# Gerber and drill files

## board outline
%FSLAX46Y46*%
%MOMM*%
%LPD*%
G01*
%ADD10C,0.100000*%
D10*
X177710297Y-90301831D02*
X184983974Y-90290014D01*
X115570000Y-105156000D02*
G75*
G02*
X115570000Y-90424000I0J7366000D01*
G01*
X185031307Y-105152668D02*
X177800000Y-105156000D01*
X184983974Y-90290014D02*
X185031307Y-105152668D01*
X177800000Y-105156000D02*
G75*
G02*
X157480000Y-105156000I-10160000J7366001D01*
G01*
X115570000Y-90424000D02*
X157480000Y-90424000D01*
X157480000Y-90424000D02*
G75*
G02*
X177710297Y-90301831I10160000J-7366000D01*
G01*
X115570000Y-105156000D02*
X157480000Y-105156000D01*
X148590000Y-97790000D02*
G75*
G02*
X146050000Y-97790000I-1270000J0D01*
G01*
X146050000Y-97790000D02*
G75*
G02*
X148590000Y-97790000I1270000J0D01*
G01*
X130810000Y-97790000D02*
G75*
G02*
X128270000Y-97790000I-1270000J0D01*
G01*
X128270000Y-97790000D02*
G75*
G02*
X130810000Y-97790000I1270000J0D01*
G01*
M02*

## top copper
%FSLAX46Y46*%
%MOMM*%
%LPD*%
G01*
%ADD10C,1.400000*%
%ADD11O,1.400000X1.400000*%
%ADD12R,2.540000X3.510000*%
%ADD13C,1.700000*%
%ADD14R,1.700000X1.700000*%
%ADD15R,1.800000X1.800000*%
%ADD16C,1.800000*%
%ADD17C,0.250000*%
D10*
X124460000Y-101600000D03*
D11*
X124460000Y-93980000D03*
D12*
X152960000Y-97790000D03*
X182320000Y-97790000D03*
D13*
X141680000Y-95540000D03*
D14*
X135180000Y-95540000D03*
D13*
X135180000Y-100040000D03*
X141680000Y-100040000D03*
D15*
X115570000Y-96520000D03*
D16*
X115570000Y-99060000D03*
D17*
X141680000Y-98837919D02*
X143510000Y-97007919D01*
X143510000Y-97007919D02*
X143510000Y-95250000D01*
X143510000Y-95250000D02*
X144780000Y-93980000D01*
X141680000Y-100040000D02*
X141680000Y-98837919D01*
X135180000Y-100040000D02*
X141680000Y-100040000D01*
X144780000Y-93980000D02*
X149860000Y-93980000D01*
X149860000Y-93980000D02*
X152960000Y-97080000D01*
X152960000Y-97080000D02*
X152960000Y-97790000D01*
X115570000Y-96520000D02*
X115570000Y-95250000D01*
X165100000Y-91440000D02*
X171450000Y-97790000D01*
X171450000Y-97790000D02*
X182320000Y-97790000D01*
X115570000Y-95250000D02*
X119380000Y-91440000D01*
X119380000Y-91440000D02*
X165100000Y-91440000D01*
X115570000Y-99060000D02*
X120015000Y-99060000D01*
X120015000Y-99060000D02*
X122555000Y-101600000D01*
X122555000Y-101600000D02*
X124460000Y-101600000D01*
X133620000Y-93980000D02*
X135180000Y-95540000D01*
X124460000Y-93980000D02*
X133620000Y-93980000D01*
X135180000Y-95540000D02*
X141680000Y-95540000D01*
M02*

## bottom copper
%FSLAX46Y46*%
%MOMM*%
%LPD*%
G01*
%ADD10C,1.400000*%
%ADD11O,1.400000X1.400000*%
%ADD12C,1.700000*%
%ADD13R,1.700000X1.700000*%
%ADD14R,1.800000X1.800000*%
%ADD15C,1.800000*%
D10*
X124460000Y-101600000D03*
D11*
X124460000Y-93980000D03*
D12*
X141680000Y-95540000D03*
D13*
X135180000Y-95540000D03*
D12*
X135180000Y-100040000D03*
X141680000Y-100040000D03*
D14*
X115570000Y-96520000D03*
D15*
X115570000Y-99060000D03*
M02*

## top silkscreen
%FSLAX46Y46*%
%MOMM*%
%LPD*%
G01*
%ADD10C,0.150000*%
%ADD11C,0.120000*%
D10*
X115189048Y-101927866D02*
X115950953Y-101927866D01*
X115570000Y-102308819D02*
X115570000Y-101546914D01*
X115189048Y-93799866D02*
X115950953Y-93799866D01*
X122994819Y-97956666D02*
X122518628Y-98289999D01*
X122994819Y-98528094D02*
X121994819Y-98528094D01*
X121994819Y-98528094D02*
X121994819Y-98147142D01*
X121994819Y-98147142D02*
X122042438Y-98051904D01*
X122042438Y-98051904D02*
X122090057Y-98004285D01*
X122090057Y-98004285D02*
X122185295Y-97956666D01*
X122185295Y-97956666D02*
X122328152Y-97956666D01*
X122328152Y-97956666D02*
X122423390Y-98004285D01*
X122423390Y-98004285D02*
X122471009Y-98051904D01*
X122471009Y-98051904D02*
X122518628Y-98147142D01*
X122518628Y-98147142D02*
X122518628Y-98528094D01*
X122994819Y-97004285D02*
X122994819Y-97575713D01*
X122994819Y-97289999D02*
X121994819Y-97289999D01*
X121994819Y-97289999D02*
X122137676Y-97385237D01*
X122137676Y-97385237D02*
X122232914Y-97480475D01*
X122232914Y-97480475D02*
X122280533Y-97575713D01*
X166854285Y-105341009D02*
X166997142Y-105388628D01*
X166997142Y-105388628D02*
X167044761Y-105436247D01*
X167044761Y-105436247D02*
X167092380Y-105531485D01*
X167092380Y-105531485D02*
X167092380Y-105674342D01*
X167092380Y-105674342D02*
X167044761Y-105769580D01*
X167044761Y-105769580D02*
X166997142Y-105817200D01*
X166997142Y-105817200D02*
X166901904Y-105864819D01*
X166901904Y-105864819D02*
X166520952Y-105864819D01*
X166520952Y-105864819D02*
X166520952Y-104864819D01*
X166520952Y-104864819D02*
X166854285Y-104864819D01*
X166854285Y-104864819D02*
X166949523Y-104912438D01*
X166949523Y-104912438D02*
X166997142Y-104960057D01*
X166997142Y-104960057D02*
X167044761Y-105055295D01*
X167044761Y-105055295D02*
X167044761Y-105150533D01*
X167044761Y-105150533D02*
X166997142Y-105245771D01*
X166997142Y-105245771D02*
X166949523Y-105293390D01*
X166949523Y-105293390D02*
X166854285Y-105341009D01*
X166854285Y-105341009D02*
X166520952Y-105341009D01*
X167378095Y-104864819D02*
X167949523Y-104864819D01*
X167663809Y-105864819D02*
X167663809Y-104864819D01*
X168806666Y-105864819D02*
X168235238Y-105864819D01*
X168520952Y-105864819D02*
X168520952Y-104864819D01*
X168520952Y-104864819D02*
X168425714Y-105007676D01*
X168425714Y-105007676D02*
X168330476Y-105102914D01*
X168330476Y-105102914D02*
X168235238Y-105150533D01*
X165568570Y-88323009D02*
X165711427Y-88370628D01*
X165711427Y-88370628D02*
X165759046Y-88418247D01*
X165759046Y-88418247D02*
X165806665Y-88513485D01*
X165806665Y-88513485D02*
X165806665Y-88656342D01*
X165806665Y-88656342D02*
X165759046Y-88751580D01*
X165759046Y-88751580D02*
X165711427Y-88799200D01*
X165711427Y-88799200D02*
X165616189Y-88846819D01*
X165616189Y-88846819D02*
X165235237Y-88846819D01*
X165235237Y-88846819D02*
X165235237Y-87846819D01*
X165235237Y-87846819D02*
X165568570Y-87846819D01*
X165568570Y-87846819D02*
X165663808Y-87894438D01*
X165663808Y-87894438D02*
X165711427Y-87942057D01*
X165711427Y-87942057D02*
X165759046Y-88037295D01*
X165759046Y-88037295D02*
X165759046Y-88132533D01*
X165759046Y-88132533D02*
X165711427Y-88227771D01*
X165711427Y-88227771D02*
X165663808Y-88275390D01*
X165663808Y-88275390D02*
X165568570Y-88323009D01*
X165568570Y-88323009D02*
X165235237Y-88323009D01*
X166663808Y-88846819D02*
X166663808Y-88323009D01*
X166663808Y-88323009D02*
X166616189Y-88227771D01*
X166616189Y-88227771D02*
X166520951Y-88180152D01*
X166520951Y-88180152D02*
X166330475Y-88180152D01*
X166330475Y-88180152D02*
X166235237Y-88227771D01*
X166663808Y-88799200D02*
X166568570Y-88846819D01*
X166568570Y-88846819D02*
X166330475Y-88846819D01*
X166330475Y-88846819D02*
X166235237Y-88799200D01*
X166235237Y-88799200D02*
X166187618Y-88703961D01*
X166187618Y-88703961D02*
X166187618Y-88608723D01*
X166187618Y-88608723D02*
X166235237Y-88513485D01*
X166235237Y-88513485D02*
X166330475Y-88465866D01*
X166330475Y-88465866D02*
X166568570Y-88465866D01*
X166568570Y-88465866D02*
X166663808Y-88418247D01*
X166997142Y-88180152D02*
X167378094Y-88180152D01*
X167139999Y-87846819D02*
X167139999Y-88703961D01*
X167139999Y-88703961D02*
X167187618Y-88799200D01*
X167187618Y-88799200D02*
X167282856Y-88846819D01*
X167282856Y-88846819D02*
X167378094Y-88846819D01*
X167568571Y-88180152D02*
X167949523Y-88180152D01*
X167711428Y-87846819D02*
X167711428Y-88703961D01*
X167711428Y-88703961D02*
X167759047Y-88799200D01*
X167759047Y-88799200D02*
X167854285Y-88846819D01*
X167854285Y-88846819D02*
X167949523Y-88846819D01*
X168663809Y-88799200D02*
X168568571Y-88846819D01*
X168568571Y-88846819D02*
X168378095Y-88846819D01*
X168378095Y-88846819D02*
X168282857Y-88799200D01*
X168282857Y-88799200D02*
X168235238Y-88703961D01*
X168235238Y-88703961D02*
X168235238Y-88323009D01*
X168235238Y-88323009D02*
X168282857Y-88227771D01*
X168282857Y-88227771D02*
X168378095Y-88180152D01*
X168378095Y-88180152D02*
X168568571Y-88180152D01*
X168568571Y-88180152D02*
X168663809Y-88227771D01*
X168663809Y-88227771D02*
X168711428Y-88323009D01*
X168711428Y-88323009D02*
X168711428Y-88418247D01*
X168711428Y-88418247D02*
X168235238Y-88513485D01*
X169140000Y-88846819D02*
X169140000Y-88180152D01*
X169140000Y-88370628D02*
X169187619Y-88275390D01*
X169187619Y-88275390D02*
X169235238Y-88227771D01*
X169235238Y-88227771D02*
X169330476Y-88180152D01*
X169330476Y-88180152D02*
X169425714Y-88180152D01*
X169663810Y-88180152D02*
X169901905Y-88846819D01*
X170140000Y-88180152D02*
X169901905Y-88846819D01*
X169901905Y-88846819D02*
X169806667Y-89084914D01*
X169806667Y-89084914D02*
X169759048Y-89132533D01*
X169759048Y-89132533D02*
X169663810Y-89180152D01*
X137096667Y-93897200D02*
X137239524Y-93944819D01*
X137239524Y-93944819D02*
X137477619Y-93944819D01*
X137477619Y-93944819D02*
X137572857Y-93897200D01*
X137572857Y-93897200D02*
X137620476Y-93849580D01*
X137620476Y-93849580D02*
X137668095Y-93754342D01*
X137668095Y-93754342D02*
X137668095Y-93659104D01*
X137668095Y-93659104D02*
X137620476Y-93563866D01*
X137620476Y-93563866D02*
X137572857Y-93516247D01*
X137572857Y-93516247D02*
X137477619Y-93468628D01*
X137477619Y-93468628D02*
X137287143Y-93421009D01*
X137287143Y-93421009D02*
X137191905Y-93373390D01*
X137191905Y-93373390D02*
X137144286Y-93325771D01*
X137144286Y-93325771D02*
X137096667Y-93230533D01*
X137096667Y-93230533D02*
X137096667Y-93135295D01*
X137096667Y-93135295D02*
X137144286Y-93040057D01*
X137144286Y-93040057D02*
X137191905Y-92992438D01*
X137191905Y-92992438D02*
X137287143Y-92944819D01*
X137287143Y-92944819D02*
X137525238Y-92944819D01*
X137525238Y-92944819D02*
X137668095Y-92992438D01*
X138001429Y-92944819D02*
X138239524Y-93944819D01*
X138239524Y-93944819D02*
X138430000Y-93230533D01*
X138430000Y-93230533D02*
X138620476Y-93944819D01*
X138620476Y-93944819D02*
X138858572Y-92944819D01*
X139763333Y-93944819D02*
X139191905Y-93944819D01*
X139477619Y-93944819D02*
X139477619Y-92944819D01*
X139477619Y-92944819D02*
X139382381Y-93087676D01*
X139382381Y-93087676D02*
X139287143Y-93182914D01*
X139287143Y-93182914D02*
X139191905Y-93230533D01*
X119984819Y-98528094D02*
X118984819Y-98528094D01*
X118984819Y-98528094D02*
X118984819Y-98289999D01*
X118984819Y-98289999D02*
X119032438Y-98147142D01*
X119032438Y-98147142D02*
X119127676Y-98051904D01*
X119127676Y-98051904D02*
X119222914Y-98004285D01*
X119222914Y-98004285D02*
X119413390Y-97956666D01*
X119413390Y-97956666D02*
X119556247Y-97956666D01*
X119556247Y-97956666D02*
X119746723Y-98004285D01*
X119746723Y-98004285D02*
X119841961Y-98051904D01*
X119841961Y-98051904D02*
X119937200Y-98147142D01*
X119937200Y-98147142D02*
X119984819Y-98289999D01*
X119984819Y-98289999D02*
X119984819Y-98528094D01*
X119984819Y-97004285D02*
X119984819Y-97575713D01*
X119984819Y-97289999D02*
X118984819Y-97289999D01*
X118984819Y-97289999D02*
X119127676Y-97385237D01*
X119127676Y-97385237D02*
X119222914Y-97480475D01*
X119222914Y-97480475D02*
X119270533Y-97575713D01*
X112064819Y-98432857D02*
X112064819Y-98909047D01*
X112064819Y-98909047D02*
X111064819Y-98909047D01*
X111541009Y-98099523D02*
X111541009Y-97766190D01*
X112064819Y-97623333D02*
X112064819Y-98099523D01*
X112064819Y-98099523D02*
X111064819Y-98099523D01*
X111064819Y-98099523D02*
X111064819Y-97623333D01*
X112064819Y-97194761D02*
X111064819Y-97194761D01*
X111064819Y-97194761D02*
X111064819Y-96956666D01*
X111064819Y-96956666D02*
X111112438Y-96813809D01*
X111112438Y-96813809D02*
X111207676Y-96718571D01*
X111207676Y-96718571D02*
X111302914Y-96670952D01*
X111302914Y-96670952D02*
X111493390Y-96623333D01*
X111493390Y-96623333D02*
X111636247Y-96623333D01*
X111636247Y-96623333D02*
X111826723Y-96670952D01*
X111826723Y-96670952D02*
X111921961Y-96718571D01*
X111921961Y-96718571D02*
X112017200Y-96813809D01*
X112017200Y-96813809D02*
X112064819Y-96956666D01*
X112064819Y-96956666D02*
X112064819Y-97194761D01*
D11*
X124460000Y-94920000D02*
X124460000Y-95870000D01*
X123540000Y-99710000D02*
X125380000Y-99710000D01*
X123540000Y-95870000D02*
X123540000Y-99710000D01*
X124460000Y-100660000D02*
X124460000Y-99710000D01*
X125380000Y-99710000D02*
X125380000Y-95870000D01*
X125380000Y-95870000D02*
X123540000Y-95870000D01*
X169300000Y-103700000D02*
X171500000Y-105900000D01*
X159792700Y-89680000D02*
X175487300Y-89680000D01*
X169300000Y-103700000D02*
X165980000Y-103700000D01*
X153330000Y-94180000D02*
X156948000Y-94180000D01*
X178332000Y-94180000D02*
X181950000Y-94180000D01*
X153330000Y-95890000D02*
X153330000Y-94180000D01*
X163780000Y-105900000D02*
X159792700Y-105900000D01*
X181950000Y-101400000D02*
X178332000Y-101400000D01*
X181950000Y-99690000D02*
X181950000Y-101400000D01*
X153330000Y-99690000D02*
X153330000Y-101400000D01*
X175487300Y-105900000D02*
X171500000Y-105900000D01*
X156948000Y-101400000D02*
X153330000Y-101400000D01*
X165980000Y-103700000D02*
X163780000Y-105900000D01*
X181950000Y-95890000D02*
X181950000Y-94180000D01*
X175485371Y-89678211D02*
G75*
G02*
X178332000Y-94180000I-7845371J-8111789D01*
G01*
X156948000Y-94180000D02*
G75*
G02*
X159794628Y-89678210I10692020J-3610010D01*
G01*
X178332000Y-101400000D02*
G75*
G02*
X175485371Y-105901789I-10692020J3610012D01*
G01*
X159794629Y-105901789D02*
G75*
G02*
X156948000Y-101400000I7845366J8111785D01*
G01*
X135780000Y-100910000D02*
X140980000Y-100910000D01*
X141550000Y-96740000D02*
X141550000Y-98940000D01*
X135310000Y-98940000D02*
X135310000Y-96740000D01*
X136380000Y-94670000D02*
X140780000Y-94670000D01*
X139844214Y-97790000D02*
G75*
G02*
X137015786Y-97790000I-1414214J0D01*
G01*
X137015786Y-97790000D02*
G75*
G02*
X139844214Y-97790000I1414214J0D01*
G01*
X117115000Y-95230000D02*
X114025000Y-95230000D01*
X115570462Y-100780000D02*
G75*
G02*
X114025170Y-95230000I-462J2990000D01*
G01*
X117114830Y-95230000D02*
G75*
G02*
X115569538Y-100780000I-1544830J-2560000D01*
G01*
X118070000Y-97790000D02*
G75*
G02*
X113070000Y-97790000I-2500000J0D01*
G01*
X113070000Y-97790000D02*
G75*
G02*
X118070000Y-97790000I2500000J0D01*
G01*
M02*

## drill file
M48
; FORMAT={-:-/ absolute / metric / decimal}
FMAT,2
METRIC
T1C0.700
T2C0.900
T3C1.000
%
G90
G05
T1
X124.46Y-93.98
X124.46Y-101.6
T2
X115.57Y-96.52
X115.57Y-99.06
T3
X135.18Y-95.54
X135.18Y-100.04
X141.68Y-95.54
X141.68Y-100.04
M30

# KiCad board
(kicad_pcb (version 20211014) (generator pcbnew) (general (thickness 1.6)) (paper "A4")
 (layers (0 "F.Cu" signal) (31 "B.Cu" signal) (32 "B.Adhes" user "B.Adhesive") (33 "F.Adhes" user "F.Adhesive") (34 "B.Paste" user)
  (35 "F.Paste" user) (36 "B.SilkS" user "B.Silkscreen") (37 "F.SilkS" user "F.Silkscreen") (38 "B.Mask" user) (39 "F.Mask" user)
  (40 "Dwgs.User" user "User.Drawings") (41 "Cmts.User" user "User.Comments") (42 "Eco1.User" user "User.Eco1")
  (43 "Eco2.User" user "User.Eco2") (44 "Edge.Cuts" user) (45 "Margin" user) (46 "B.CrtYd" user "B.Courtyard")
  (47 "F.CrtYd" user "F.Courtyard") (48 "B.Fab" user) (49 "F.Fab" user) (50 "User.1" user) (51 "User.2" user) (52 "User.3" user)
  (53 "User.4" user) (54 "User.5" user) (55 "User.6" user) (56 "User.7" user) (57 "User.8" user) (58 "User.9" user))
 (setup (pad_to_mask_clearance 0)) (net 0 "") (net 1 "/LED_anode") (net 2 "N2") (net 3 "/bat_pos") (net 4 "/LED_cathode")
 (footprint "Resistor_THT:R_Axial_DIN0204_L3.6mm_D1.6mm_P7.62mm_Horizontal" (layer "F.Cu") (at 124.46 101.6 90)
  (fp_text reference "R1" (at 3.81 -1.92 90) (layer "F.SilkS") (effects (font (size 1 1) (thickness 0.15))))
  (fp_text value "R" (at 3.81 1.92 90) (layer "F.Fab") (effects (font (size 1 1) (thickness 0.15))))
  (fp_line (start 6.68 0) (end 5.73 0) (layer "F.SilkS") (width 0.12))
  (fp_line (start 1.89 -0.92) (end 1.89 0.92) (layer "F.SilkS") (width 0.12))
  (fp_line (start 5.73 -0.92) (end 1.89 -0.92) (layer "F.SilkS") (width 0.12))
  (fp_line (start 0.94 0) (end 1.89 0) (layer "F.SilkS") (width 0.12))
  (fp_line (start 1.89 0.92) (end 5.73 0.92) (layer "F.SilkS") (width 0.12))
  (fp_line (start 5.73 0.92) (end 5.73 -0.92) (layer "F.SilkS") (width 0.12))
  (pad "1" thru_hole circle (at 0 0 90) (size 1.4 1.4) (drill 0.7) (layers *.Cu *.Mask) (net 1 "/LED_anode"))
  (pad "2" thru_hole oval (at 7.62 0 90) (size 1.4 1.4) (drill 0.7) (layers *.Cu *.Mask) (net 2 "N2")))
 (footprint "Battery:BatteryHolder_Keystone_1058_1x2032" (layer "F.Cu") (at 167.64 97.79)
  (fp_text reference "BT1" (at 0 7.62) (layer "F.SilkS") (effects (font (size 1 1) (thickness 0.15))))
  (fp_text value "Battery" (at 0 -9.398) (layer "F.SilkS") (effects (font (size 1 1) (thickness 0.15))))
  (fp_line (start 1.66 5.91) (end 3.86 8.11) (layer "F.SilkS") (width 0.12))
  (fp_line (start -7.8473 -8.11) (end 7.8473 -8.11) (layer "F.SilkS") (width 0.12))
  (fp_line (start 1.66 5.91) (end -1.66 5.91) (layer "F.SilkS") (width 0.12))
  (fp_line (start -14.31 -3.61) (end -10.692 -3.61) (layer "F.SilkS") (width 0.12))
  (fp_line (start 10.692 -3.61) (end 14.31 -3.61) (layer "F.SilkS") (width 0.12))
  (fp_line (start -14.31 -1.9) (end -14.31 -3.61) (layer "F.SilkS") (width 0.12))
  (fp_line (start -3.86 8.11) (end -7.8473 8.11) (layer "F.SilkS") (width 0.12))
  (fp_line (start 14.31 3.61) (end 10.692 3.61) (layer "F.SilkS") (width 0.12))
  (fp_line (start 14.31 1.9) (end 14.31 3.61) (layer "F.SilkS") (width 0.12))
  (fp_line (start -14.31 1.9) (end -14.31 3.61) (layer "F.SilkS") (width 0.12))
  (fp_line (start 7.8473 8.11) (end 3.86 8.11) (layer "F.SilkS") (width 0.12))
  (fp_line (start -10.692 3.61) (end -14.31 3.61) (layer "F.SilkS") (width 0.12))
  (fp_line (start -1.66 5.91) (end -3.86 8.11) (layer "F.SilkS") (width 0.12))
  (fp_line (start 14.31 -1.9) (end 14.31 -3.61) (layer "F.SilkS") (width 0.12))
  (fp_arc (start 7.845371 -8.111789) (mid 9.538085 -6.031244) (end 10.692 -3.61) (layer "F.SilkS") (width 0.12))
  (fp_arc (start -10.692 -3.61) (mid -9.538084 -6.031244) (end -7.845371 -8.111789) (layer "F.SilkS") (width 0.12))
  (fp_arc (start 10.692 3.61) (mid 9.538084 6.031244) (end 7.845371 8.111789) (layer "F.SilkS") (width 0.12))
  (fp_arc (start -7.845371 8.111789) (mid -9.538085 6.031244) (end -10.692 3.61) (layer "F.SilkS") (width 0.12))
  (pad "1" smd rect (at -14.68 0) (size 2.54 3.51) (layers "F.Cu" "F.Paste" "F.Mask") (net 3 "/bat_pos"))
  (pad "2" smd rect (at 14.68 0) (size 2.54 3.51) (layers "F.Cu" "F.Paste" "F.Mask") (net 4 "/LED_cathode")))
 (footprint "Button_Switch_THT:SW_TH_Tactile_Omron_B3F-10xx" (layer "F.Cu") (at 135.18 95.54)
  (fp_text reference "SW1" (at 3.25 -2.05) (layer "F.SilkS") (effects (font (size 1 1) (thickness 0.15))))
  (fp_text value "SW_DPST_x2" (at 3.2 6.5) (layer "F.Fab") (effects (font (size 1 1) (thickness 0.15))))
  (fp_line (start 0.6 5.37) (end 5.8 5.37) (layer "F.SilkS") (width 0.12))
  (fp_line (start 6.37 1.2) (end 6.37 3.4) (layer "F.SilkS") (width 0.12))
  (fp_line (start 0.13 3.4) (end 0.13 1.2) (layer "F.SilkS") (width 0.12))
  (fp_line (start 1.2 -0.87) (end 5.6 -0.87) (layer "F.SilkS") (width 0.12))
  (fp_circle (center 3.25 2.25) (end 4.25 3.25) (layer "F.SilkS") (width 0.12) (fill none))
  (pad "1" thru_hole circle (at 6.5 0) (size 1.7 1.7) (drill 1) (layers *.Cu *.Mask) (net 2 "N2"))
  (pad "1" thru_hole rect (at 0 0) (size 1.7 1.7) (drill 1) (layers *.Cu *.Mask) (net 2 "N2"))
  (pad "2" thru_hole circle (at 0 4.5) (size 1.7 1.7) (drill 1) (layers *.Cu *.Mask) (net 3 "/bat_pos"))
  (pad "2" thru_hole circle (at 6.5 4.5) (size 1.7 1.7) (drill 1) (layers *.Cu *.Mask) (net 3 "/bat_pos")))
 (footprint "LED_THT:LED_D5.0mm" (layer "F.Cu") (at 115.57 96.52 -90)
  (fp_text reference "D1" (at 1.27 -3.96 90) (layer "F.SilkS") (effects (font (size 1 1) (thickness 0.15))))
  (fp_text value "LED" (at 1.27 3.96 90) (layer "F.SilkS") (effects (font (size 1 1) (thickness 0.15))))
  (fp_line (start -1.29 -1.545) (end -1.29 1.545) (layer "F.SilkS") (width 0.12))
  (fp_arc (start 4.26 -0.000462) (mid 2.072002 2.880433) (end -1.29 1.54483) (layer "F.SilkS") (width 0.12))
  (fp_arc (start -1.29 -1.54483) (mid 2.072002 -2.880433) (end 4.26 0.000462) (layer "F.SilkS") (width 0.12))
  (fp_circle (center 1.27 0) (end 3.77 0) (layer "F.SilkS") (width 0.12) (fill none))
  (pad "1" thru_hole rect (at 0 0 270) (size 1.8 1.8) (drill 0.9) (layers *.Cu *.Mask) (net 4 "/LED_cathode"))
  (pad "2" thru_hole circle (at 2.54 0 270) (size 1.8 1.8) (drill 0.9) (layers *.Cu *.Mask) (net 1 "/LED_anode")))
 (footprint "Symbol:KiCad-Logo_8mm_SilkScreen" (layer "B.Cu") (at 167.64 97.536 180)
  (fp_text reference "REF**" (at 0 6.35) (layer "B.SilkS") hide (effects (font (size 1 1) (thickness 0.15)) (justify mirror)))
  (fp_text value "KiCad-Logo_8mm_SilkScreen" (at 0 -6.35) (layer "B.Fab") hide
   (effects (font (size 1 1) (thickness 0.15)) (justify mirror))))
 (gr_line (start 177.710297 90.301831) (end 184.983974 90.290014) (layer "Edge.Cuts") (width 0.1))
 (gr_arc (start 115.57 105.156) (mid 108.204 97.79) (end 115.57 90.424) (layer "Edge.Cuts") (width 0.1))
 (gr_line (start 185.031307 105.152668) (end 177.8 105.156) (layer "Edge.Cuts") (width 0.1))
 (gr_line (start 184.983974 90.290014) (end 185.031307 105.152668) (layer "Edge.Cuts") (width 0.1))
 (gr_arc (start 177.8 105.156) (mid 167.64 110.339245) (end 157.48 105.156) (layer "Edge.Cuts") (width 0.1))
 (gr_line (start 115.57 90.424) (end 157.48 90.424) (layer "Edge.Cuts") (width 0.1))
 (gr_arc (start 157.48 90.424) (mid 167.564218 85.240984) (end 177.710297 90.301831) (layer "Edge.Cuts") (width 0.1))
 (gr_line (start 115.57 105.156) (end 157.48 105.156) (layer "Edge.Cuts") (width 0.1))
 (gr_circle (center 147.32 97.79) (end 146.05 97.79) (layer "Edge.Cuts") (width 0.1) (fill none))
 (gr_circle (center 129.54 97.79) (end 128.27 97.79) (layer "Edge.Cuts") (width 0.1) (fill none))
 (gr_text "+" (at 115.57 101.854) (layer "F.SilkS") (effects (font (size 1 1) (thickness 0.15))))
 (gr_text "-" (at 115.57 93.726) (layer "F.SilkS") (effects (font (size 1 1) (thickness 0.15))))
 (segment (start 141.68 98.837919) (end 143.51 97.007919) (width 0.25) (layer "F.Cu") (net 3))
 (segment (start 143.51 97.007919) (end 143.51 95.25) (width 0.25) (layer "F.Cu") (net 3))
 (segment (start 143.51 95.25) (end 144.78 93.98) (width 0.25) (layer "F.Cu") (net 3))
 (segment (start 141.68 100.04) (end 141.68 98.837919) (width 0.25) (layer "F.Cu") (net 3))
 (segment (start 135.18 100.04) (end 141.68 100.04) (width 0.25) (layer "F.Cu") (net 3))
 (segment (start 144.78 93.98) (end 149.86 93.98) (width 0.25) (layer "F.Cu") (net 3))
 (segment (start 149.86 93.98) (end 152.96 97.08) (width 0.25) (layer "F.Cu") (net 3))
 (segment (start 152.96 97.08) (end 152.96 97.79) (width 0.25) (layer "F.Cu") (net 3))
 (segment (start 115.57 96.52) (end 115.57 95.25) (width 0.25) (layer "F.Cu") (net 4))
 (segment (start 165.1 91.44) (end 171.45 97.79) (width 0.25) (layer "F.Cu") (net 4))
 (segment (start 171.45 97.79) (end 182.32 97.79) (width 0.25) (layer "F.Cu") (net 4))
 (segment (start 115.57 95.25) (end 119.38 91.44) (width 0.25) (layer "F.Cu") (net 4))
 (segment (start 119.38 91.44) (end 165.1 91.44) (width 0.25) (layer "F.Cu") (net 4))
 (segment (start 115.57 99.06) (end 120.015 99.06) (width 0.25) (layer "F.Cu") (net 1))
 (segment (start 120.015 99.06) (end 122.555 101.6) (width 0.25) (layer "F.Cu") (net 1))
 (segment (start 122.555 101.6) (end 124.46 101.6) (width 0.25) (layer "F.Cu") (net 1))
 (segment (start 133.62 93.98) (end 135.18 95.54) (width 0.25) (layer "F.Cu") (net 2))
 (segment (start 124.46 93.98) (end 133.62 93.98) (width 0.25) (layer "F.Cu") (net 2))
 (segment (start 135.18 95.54) (end 141.68 95.54) (width 0.25) (layer "F.Cu") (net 2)))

